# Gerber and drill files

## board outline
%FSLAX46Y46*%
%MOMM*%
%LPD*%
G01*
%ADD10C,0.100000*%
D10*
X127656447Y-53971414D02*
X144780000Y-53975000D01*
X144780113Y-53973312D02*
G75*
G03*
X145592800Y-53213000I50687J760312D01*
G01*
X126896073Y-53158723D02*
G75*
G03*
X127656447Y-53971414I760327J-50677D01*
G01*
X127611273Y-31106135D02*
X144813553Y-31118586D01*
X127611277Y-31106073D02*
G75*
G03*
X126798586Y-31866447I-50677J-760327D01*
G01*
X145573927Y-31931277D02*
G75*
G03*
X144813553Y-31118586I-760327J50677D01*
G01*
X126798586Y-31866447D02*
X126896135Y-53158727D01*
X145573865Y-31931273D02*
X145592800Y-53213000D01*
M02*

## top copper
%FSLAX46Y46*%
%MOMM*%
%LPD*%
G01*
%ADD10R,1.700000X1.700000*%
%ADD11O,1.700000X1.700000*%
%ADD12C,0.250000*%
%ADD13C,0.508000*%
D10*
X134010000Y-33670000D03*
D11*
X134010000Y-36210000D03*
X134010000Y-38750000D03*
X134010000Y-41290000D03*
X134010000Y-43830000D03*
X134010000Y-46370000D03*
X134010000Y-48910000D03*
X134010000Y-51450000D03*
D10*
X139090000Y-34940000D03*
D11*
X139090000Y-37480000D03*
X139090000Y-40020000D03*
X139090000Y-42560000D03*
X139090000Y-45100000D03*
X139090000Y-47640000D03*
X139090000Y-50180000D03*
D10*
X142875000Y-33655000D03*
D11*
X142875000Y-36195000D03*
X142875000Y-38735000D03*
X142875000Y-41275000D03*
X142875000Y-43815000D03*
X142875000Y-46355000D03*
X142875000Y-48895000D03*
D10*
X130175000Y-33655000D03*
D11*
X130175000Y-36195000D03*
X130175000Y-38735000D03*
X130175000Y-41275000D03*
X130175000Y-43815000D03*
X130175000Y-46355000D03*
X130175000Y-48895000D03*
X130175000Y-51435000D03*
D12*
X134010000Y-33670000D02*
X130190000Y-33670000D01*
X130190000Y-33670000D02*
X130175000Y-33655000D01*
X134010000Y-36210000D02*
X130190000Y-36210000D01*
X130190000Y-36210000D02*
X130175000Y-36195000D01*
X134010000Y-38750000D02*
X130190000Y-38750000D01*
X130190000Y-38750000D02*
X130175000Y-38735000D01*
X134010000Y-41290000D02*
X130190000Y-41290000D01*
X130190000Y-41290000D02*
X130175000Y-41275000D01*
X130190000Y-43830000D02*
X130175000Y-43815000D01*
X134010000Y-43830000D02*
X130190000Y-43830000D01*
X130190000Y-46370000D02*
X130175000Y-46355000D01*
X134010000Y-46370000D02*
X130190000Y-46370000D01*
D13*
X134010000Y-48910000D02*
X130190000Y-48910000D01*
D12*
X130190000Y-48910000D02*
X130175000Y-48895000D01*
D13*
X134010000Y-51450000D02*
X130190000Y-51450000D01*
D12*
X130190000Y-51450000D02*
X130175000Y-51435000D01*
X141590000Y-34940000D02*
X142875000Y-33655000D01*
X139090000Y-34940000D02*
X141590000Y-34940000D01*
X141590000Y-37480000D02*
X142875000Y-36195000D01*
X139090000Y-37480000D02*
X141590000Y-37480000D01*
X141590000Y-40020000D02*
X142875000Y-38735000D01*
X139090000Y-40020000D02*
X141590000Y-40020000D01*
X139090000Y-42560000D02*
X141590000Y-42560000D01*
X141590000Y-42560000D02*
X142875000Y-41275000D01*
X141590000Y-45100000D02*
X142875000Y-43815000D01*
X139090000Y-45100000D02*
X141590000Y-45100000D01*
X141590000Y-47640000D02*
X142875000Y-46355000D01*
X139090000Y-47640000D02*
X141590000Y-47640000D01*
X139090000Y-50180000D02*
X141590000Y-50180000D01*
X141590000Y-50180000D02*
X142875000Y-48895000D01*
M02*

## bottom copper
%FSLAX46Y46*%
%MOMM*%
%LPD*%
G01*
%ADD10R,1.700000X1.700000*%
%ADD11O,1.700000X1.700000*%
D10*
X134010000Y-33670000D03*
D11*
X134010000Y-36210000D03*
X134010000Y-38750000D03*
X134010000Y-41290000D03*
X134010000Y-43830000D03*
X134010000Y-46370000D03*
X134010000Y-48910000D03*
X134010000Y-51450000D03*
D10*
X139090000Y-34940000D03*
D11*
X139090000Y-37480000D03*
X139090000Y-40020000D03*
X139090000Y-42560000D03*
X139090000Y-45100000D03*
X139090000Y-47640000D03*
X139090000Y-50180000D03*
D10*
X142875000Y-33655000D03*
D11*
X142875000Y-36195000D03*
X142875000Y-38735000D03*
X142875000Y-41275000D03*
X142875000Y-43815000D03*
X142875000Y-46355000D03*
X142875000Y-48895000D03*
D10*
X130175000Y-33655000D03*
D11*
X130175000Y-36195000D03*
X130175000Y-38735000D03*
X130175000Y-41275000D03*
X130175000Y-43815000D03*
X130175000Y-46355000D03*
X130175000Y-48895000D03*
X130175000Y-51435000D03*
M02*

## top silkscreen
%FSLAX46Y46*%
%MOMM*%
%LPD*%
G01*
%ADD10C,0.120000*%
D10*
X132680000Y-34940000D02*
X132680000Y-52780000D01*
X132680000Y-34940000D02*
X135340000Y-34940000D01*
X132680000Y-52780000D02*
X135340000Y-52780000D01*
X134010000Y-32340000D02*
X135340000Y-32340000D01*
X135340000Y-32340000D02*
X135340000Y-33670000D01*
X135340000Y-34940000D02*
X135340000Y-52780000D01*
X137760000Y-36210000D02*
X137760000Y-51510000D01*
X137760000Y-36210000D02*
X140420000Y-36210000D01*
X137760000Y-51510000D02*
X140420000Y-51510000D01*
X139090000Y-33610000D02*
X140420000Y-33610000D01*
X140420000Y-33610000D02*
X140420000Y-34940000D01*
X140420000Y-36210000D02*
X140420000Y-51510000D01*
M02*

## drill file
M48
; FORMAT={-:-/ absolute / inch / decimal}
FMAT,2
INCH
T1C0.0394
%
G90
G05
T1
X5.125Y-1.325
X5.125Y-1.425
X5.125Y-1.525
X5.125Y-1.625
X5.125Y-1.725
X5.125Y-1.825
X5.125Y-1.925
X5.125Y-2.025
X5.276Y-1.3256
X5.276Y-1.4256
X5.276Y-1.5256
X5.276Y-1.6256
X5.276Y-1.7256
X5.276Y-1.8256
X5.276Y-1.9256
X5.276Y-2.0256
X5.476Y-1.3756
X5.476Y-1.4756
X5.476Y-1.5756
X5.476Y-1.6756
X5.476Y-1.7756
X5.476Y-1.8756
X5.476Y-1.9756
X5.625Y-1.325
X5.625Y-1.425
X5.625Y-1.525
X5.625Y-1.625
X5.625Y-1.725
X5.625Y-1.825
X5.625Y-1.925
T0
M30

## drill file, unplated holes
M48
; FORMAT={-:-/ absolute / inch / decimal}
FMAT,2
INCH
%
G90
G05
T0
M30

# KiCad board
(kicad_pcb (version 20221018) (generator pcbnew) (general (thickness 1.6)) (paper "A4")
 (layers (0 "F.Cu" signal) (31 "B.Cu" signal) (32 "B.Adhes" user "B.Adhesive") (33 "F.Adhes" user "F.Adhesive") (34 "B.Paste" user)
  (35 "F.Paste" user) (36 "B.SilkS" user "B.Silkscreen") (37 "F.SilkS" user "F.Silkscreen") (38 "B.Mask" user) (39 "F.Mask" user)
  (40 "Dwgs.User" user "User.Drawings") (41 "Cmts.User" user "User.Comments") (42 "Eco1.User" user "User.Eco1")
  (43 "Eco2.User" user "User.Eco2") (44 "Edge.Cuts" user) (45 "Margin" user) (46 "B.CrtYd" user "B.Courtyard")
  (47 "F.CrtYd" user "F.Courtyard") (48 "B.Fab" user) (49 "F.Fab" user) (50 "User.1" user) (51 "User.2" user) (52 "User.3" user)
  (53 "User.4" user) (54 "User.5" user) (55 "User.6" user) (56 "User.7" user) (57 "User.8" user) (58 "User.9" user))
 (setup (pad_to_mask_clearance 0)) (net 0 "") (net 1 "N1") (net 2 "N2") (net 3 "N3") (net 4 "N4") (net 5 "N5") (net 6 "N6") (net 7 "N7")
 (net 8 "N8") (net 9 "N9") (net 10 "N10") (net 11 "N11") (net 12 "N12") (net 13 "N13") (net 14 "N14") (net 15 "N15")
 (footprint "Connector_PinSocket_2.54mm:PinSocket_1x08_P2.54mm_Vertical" (layer "F.Cu") (at 134.01 33.67)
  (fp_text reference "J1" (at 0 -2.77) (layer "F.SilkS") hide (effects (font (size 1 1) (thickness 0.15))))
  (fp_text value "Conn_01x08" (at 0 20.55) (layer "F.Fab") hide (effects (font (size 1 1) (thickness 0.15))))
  (fp_line (start -1.33 1.27) (end -1.33 19.11) (stroke (width 0.12) (type solid)) (layer "F.SilkS"))
  (fp_line (start -1.33 1.27) (end 1.33 1.27) (stroke (width 0.12) (type solid)) (layer "F.SilkS"))
  (fp_line (start -1.33 19.11) (end 1.33 19.11) (stroke (width 0.12) (type solid)) (layer "F.SilkS"))
  (fp_line (start 0 -1.33) (end 1.33 -1.33) (stroke (width 0.12) (type solid)) (layer "F.SilkS"))
  (fp_line (start 1.33 -1.33) (end 1.33 0) (stroke (width 0.12) (type solid)) (layer "F.SilkS"))
  (fp_line (start 1.33 1.27) (end 1.33 19.11) (stroke (width 0.12) (type solid)) (layer "F.SilkS"))
  (pad "1" thru_hole rect (at 0 0) (size 1.7 1.7) (drill 1) (layers "*.Cu" "*.Mask") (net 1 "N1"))
  (pad "2" thru_hole oval (at 0 2.54) (size 1.7 1.7) (drill 1) (layers "*.Cu" "*.Mask") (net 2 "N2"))
  (pad "3" thru_hole oval (at 0 5.08) (size 1.7 1.7) (drill 1) (layers "*.Cu" "*.Mask") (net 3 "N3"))
  (pad "4" thru_hole oval (at 0 7.62) (size 1.7 1.7) (drill 1) (layers "*.Cu" "*.Mask") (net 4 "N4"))
  (pad "5" thru_hole oval (at 0 10.16) (size 1.7 1.7) (drill 1) (layers "*.Cu" "*.Mask") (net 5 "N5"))
  (pad "6" thru_hole oval (at 0 12.7) (size 1.7 1.7) (drill 1) (layers "*.Cu" "*.Mask") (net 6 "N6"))
  (pad "7" thru_hole oval (at 0 15.24) (size 1.7 1.7) (drill 1) (layers "*.Cu" "*.Mask") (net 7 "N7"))
  (pad "8" thru_hole oval (at 0 17.78) (size 1.7 1.7) (drill 1) (layers "*.Cu" "*.Mask") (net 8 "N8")))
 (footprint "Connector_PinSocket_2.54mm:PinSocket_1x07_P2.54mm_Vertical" (layer "F.Cu") (at 139.09 34.94)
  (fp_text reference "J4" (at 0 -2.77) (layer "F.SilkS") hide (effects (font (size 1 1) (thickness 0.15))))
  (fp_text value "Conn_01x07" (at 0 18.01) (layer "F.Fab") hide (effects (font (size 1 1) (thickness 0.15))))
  (fp_line (start -1.33 1.27) (end -1.33 16.57) (stroke (width 0.12) (type solid)) (layer "F.SilkS"))
  (fp_line (start -1.33 1.27) (end 1.33 1.27) (stroke (width 0.12) (type solid)) (layer "F.SilkS"))
  (fp_line (start -1.33 16.57) (end 1.33 16.57) (stroke (width 0.12) (type solid)) (layer "F.SilkS"))
  (fp_line (start 0 -1.33) (end 1.33 -1.33) (stroke (width 0.12) (type solid)) (layer "F.SilkS"))
  (fp_line (start 1.33 -1.33) (end 1.33 0) (stroke (width 0.12) (type solid)) (layer "F.SilkS"))
  (fp_line (start 1.33 1.27) (end 1.33 16.57) (stroke (width 0.12) (type solid)) (layer "F.SilkS"))
  (pad "1" thru_hole rect (at 0 0) (size 1.7 1.7) (drill 1) (layers "*.Cu" "*.Mask") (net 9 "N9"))
  (pad "2" thru_hole oval (at 0 2.54) (size 1.7 1.7) (drill 1) (layers "*.Cu" "*.Mask") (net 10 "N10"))
  (pad "3" thru_hole oval (at 0 5.08) (size 1.7 1.7) (drill 1) (layers "*.Cu" "*.Mask") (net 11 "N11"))
  (pad "4" thru_hole oval (at 0 7.62) (size 1.7 1.7) (drill 1) (layers "*.Cu" "*.Mask") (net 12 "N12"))
  (pad "5" thru_hole oval (at 0 10.16) (size 1.7 1.7) (drill 1) (layers "*.Cu" "*.Mask") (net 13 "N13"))
  (pad "6" thru_hole oval (at 0 12.7) (size 1.7 1.7) (drill 1) (layers "*.Cu" "*.Mask") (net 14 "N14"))
  (pad "7" thru_hole oval (at 0 15.24) (size 1.7 1.7) (drill 1) (layers "*.Cu" "*.Mask") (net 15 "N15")))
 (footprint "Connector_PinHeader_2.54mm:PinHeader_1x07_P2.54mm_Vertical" (layer "B.Cu") (at 142.875 33.655 180)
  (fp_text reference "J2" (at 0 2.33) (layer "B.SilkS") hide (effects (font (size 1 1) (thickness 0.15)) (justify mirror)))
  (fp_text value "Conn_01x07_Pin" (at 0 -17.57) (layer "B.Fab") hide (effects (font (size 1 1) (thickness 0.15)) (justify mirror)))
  (pad "1" thru_hole rect (at 0 0 180) (size 1.7 1.7) (drill 1) (layers "*.Cu" "*.Mask") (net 9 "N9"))
  (pad "2" thru_hole oval (at 0 -2.54 180) (size 1.7 1.7) (drill 1) (layers "*.Cu" "*.Mask") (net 10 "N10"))
  (pad "3" thru_hole oval (at 0 -5.08 180) (size 1.7 1.7) (drill 1) (layers "*.Cu" "*.Mask") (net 11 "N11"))
  (pad "4" thru_hole oval (at 0 -7.62 180) (size 1.7 1.7) (drill 1) (layers "*.Cu" "*.Mask") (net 12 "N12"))
  (pad "5" thru_hole oval (at 0 -10.16 180) (size 1.7 1.7) (drill 1) (layers "*.Cu" "*.Mask") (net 13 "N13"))
  (pad "6" thru_hole oval (at 0 -12.7 180) (size 1.7 1.7) (drill 1) (layers "*.Cu" "*.Mask") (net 14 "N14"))
  (pad "7" thru_hole oval (at 0 -15.24 180) (size 1.7 1.7) (drill 1) (layers "*.Cu" "*.Mask") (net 15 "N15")))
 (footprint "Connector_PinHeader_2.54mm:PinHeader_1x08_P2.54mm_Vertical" (layer "B.Cu") (at 130.175 33.655 180)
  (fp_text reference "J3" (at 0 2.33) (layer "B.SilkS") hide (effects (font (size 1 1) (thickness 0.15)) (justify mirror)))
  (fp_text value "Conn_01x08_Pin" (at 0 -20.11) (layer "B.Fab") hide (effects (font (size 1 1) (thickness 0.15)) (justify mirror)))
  (pad "1" thru_hole rect (at 0 0 180) (size 1.7 1.7) (drill 1) (layers "*.Cu" "*.Mask") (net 1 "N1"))
  (pad "2" thru_hole oval (at 0 -2.54 180) (size 1.7 1.7) (drill 1) (layers "*.Cu" "*.Mask") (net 2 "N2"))
  (pad "3" thru_hole oval (at 0 -5.08 180) (size 1.7 1.7) (drill 1) (layers "*.Cu" "*.Mask") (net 3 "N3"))
  (pad "4" thru_hole oval (at 0 -7.62 180) (size 1.7 1.7) (drill 1) (layers "*.Cu" "*.Mask") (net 4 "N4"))
  (pad "5" thru_hole oval (at 0 -10.16 180) (size 1.7 1.7) (drill 1) (layers "*.Cu" "*.Mask") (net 5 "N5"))
  (pad "6" thru_hole oval (at 0 -12.7 180) (size 1.7 1.7) (drill 1) (layers "*.Cu" "*.Mask") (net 6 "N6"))
  (pad "7" thru_hole oval (at 0 -15.24 180) (size 1.7 1.7) (drill 1) (layers "*.Cu" "*.Mask") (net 7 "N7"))
  (pad "8" thru_hole oval (at 0 -17.78 180) (size 1.7 1.7) (drill 1) (layers "*.Cu" "*.Mask") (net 8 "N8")))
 (gr_line (start 127.656447 53.971414) (end 144.78 53.975) (stroke (width 0.1) (type default)) (layer "Edge.Cuts"))
 (gr_arc (start 145.5928 53.213) (mid 145.351386 53.769447) (end 144.780113 53.973312) (stroke (width 0.1) (type default))
  (layer "Edge.Cuts"))
 (gr_arc (start 127.656447 53.971414) (mid 127.1 53.73) (end 126.896135 53.158727) (stroke (width 0.1) (type default)) (layer "Edge.Cuts"))
 (gr_line (start 127.611273 31.106135) (end 144.813553 31.118586) (stroke (width 0.1) (type default)) (layer "Edge.Cuts"))
 (gr_arc (start 126.798586 31.866447) (mid 127.04 31.31) (end 127.611273 31.106135) (stroke (width 0.1) (type default)) (layer "Edge.Cuts"))
 (gr_arc (start 144.813553 31.118586) (mid 145.37 31.36) (end 145.573865 31.931273) (stroke (width 0.1) (type default)) (layer "Edge.Cuts"))
 (gr_line (start 126.798586 31.866447) (end 126.896135 53.158727) (stroke (width 0.1) (type default)) (layer "Edge.Cuts"))
 (gr_line (start 145.573865 31.931273) (end 145.5928 53.213) (stroke (width 0.1) (type default)) (layer "Edge.Cuts"))
 (segment (start 134.01 33.67) (end 130.19 33.67) (width 0.25) (layer "F.Cu") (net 1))
 (segment (start 130.19 33.67) (end 130.175 33.655) (width 0.25) (layer "F.Cu") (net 1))
 (segment (start 134.01 36.21) (end 130.19 36.21) (width 0.25) (layer "F.Cu") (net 2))
 (segment (start 130.19 36.21) (end 130.175 36.195) (width 0.25) (layer "F.Cu") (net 2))
 (segment (start 134.01 38.75) (end 130.19 38.75) (width 0.25) (layer "F.Cu") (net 3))
 (segment (start 130.19 38.75) (end 130.175 38.735) (width 0.25) (layer "F.Cu") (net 3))
 (segment (start 134.01 41.29) (end 130.19 41.29) (width 0.25) (layer "F.Cu") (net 4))
 (segment (start 130.19 41.29) (end 130.175 41.275) (width 0.25) (layer "F.Cu") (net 4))
 (segment (start 130.19 43.83) (end 130.175 43.815) (width 0.25) (layer "F.Cu") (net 5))
 (segment (start 134.01 43.83) (end 130.19 43.83) (width 0.25) (layer "F.Cu") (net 5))
 (segment (start 130.19 46.37) (end 130.175 46.355) (width 0.25) (layer "F.Cu") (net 6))
 (segment (start 134.01 46.37) (end 130.19 46.37) (width 0.25) (layer "F.Cu") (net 6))
 (segment (start 134.01 48.91) (end 130.19 48.91) (width 0.508) (layer "F.Cu") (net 7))
 (segment (start 130.19 48.91) (end 130.175 48.895) (width 0.25) (layer "F.Cu") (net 7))
 (segment (start 134.01 51.45) (end 130.19 51.45) (width 0.508) (layer "F.Cu") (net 8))
 (segment (start 130.19 51.45) (end 130.175 51.435) (width 0.25) (layer "F.Cu") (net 8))
 (segment (start 141.59 34.94) (end 142.875 33.655) (width 0.25) (layer "F.Cu") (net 9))
 (segment (start 139.09 34.94) (end 141.59 34.94) (width 0.25) (layer "F.Cu") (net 9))
 (segment (start 141.59 37.48) (end 142.875 36.195) (width 0.25) (layer "F.Cu") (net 10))
 (segment (start 139.09 37.48) (end 141.59 37.48) (width 0.25) (layer "F.Cu") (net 10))
 (segment (start 141.59 40.02) (end 142.875 38.735) (width 0.25) (layer "F.Cu") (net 11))
 (segment (start 139.09 40.02) (end 141.59 40.02) (width 0.25) (layer "F.Cu") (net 11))
 (segment (start 139.09 42.56) (end 141.59 42.56) (width 0.25) (layer "F.Cu") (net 12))
 (segment (start 141.59 42.56) (end 142.875 41.275) (width 0.25) (layer "F.Cu") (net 12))
 (segment (start 141.59 45.1) (end 142.875 43.815) (width 0.25) (layer "F.Cu") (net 13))
 (segment (start 139.09 45.1) (end 141.59 45.1) (width 0.25) (layer "F.Cu") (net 13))
 (segment (start 141.59 47.64) (end 142.875 46.355) (width 0.25) (layer "F.Cu") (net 14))
 (segment (start 139.09 47.64) (end 141.59 47.64) (width 0.25) (layer "F.Cu") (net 14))
 (segment (start 139.09 50.18) (end 141.59 50.18) (width 0.25) (layer "F.Cu") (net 15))
 (segment (start 141.59 50.18) (end 142.875 48.895) (width 0.25) (layer "F.Cu") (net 15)))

